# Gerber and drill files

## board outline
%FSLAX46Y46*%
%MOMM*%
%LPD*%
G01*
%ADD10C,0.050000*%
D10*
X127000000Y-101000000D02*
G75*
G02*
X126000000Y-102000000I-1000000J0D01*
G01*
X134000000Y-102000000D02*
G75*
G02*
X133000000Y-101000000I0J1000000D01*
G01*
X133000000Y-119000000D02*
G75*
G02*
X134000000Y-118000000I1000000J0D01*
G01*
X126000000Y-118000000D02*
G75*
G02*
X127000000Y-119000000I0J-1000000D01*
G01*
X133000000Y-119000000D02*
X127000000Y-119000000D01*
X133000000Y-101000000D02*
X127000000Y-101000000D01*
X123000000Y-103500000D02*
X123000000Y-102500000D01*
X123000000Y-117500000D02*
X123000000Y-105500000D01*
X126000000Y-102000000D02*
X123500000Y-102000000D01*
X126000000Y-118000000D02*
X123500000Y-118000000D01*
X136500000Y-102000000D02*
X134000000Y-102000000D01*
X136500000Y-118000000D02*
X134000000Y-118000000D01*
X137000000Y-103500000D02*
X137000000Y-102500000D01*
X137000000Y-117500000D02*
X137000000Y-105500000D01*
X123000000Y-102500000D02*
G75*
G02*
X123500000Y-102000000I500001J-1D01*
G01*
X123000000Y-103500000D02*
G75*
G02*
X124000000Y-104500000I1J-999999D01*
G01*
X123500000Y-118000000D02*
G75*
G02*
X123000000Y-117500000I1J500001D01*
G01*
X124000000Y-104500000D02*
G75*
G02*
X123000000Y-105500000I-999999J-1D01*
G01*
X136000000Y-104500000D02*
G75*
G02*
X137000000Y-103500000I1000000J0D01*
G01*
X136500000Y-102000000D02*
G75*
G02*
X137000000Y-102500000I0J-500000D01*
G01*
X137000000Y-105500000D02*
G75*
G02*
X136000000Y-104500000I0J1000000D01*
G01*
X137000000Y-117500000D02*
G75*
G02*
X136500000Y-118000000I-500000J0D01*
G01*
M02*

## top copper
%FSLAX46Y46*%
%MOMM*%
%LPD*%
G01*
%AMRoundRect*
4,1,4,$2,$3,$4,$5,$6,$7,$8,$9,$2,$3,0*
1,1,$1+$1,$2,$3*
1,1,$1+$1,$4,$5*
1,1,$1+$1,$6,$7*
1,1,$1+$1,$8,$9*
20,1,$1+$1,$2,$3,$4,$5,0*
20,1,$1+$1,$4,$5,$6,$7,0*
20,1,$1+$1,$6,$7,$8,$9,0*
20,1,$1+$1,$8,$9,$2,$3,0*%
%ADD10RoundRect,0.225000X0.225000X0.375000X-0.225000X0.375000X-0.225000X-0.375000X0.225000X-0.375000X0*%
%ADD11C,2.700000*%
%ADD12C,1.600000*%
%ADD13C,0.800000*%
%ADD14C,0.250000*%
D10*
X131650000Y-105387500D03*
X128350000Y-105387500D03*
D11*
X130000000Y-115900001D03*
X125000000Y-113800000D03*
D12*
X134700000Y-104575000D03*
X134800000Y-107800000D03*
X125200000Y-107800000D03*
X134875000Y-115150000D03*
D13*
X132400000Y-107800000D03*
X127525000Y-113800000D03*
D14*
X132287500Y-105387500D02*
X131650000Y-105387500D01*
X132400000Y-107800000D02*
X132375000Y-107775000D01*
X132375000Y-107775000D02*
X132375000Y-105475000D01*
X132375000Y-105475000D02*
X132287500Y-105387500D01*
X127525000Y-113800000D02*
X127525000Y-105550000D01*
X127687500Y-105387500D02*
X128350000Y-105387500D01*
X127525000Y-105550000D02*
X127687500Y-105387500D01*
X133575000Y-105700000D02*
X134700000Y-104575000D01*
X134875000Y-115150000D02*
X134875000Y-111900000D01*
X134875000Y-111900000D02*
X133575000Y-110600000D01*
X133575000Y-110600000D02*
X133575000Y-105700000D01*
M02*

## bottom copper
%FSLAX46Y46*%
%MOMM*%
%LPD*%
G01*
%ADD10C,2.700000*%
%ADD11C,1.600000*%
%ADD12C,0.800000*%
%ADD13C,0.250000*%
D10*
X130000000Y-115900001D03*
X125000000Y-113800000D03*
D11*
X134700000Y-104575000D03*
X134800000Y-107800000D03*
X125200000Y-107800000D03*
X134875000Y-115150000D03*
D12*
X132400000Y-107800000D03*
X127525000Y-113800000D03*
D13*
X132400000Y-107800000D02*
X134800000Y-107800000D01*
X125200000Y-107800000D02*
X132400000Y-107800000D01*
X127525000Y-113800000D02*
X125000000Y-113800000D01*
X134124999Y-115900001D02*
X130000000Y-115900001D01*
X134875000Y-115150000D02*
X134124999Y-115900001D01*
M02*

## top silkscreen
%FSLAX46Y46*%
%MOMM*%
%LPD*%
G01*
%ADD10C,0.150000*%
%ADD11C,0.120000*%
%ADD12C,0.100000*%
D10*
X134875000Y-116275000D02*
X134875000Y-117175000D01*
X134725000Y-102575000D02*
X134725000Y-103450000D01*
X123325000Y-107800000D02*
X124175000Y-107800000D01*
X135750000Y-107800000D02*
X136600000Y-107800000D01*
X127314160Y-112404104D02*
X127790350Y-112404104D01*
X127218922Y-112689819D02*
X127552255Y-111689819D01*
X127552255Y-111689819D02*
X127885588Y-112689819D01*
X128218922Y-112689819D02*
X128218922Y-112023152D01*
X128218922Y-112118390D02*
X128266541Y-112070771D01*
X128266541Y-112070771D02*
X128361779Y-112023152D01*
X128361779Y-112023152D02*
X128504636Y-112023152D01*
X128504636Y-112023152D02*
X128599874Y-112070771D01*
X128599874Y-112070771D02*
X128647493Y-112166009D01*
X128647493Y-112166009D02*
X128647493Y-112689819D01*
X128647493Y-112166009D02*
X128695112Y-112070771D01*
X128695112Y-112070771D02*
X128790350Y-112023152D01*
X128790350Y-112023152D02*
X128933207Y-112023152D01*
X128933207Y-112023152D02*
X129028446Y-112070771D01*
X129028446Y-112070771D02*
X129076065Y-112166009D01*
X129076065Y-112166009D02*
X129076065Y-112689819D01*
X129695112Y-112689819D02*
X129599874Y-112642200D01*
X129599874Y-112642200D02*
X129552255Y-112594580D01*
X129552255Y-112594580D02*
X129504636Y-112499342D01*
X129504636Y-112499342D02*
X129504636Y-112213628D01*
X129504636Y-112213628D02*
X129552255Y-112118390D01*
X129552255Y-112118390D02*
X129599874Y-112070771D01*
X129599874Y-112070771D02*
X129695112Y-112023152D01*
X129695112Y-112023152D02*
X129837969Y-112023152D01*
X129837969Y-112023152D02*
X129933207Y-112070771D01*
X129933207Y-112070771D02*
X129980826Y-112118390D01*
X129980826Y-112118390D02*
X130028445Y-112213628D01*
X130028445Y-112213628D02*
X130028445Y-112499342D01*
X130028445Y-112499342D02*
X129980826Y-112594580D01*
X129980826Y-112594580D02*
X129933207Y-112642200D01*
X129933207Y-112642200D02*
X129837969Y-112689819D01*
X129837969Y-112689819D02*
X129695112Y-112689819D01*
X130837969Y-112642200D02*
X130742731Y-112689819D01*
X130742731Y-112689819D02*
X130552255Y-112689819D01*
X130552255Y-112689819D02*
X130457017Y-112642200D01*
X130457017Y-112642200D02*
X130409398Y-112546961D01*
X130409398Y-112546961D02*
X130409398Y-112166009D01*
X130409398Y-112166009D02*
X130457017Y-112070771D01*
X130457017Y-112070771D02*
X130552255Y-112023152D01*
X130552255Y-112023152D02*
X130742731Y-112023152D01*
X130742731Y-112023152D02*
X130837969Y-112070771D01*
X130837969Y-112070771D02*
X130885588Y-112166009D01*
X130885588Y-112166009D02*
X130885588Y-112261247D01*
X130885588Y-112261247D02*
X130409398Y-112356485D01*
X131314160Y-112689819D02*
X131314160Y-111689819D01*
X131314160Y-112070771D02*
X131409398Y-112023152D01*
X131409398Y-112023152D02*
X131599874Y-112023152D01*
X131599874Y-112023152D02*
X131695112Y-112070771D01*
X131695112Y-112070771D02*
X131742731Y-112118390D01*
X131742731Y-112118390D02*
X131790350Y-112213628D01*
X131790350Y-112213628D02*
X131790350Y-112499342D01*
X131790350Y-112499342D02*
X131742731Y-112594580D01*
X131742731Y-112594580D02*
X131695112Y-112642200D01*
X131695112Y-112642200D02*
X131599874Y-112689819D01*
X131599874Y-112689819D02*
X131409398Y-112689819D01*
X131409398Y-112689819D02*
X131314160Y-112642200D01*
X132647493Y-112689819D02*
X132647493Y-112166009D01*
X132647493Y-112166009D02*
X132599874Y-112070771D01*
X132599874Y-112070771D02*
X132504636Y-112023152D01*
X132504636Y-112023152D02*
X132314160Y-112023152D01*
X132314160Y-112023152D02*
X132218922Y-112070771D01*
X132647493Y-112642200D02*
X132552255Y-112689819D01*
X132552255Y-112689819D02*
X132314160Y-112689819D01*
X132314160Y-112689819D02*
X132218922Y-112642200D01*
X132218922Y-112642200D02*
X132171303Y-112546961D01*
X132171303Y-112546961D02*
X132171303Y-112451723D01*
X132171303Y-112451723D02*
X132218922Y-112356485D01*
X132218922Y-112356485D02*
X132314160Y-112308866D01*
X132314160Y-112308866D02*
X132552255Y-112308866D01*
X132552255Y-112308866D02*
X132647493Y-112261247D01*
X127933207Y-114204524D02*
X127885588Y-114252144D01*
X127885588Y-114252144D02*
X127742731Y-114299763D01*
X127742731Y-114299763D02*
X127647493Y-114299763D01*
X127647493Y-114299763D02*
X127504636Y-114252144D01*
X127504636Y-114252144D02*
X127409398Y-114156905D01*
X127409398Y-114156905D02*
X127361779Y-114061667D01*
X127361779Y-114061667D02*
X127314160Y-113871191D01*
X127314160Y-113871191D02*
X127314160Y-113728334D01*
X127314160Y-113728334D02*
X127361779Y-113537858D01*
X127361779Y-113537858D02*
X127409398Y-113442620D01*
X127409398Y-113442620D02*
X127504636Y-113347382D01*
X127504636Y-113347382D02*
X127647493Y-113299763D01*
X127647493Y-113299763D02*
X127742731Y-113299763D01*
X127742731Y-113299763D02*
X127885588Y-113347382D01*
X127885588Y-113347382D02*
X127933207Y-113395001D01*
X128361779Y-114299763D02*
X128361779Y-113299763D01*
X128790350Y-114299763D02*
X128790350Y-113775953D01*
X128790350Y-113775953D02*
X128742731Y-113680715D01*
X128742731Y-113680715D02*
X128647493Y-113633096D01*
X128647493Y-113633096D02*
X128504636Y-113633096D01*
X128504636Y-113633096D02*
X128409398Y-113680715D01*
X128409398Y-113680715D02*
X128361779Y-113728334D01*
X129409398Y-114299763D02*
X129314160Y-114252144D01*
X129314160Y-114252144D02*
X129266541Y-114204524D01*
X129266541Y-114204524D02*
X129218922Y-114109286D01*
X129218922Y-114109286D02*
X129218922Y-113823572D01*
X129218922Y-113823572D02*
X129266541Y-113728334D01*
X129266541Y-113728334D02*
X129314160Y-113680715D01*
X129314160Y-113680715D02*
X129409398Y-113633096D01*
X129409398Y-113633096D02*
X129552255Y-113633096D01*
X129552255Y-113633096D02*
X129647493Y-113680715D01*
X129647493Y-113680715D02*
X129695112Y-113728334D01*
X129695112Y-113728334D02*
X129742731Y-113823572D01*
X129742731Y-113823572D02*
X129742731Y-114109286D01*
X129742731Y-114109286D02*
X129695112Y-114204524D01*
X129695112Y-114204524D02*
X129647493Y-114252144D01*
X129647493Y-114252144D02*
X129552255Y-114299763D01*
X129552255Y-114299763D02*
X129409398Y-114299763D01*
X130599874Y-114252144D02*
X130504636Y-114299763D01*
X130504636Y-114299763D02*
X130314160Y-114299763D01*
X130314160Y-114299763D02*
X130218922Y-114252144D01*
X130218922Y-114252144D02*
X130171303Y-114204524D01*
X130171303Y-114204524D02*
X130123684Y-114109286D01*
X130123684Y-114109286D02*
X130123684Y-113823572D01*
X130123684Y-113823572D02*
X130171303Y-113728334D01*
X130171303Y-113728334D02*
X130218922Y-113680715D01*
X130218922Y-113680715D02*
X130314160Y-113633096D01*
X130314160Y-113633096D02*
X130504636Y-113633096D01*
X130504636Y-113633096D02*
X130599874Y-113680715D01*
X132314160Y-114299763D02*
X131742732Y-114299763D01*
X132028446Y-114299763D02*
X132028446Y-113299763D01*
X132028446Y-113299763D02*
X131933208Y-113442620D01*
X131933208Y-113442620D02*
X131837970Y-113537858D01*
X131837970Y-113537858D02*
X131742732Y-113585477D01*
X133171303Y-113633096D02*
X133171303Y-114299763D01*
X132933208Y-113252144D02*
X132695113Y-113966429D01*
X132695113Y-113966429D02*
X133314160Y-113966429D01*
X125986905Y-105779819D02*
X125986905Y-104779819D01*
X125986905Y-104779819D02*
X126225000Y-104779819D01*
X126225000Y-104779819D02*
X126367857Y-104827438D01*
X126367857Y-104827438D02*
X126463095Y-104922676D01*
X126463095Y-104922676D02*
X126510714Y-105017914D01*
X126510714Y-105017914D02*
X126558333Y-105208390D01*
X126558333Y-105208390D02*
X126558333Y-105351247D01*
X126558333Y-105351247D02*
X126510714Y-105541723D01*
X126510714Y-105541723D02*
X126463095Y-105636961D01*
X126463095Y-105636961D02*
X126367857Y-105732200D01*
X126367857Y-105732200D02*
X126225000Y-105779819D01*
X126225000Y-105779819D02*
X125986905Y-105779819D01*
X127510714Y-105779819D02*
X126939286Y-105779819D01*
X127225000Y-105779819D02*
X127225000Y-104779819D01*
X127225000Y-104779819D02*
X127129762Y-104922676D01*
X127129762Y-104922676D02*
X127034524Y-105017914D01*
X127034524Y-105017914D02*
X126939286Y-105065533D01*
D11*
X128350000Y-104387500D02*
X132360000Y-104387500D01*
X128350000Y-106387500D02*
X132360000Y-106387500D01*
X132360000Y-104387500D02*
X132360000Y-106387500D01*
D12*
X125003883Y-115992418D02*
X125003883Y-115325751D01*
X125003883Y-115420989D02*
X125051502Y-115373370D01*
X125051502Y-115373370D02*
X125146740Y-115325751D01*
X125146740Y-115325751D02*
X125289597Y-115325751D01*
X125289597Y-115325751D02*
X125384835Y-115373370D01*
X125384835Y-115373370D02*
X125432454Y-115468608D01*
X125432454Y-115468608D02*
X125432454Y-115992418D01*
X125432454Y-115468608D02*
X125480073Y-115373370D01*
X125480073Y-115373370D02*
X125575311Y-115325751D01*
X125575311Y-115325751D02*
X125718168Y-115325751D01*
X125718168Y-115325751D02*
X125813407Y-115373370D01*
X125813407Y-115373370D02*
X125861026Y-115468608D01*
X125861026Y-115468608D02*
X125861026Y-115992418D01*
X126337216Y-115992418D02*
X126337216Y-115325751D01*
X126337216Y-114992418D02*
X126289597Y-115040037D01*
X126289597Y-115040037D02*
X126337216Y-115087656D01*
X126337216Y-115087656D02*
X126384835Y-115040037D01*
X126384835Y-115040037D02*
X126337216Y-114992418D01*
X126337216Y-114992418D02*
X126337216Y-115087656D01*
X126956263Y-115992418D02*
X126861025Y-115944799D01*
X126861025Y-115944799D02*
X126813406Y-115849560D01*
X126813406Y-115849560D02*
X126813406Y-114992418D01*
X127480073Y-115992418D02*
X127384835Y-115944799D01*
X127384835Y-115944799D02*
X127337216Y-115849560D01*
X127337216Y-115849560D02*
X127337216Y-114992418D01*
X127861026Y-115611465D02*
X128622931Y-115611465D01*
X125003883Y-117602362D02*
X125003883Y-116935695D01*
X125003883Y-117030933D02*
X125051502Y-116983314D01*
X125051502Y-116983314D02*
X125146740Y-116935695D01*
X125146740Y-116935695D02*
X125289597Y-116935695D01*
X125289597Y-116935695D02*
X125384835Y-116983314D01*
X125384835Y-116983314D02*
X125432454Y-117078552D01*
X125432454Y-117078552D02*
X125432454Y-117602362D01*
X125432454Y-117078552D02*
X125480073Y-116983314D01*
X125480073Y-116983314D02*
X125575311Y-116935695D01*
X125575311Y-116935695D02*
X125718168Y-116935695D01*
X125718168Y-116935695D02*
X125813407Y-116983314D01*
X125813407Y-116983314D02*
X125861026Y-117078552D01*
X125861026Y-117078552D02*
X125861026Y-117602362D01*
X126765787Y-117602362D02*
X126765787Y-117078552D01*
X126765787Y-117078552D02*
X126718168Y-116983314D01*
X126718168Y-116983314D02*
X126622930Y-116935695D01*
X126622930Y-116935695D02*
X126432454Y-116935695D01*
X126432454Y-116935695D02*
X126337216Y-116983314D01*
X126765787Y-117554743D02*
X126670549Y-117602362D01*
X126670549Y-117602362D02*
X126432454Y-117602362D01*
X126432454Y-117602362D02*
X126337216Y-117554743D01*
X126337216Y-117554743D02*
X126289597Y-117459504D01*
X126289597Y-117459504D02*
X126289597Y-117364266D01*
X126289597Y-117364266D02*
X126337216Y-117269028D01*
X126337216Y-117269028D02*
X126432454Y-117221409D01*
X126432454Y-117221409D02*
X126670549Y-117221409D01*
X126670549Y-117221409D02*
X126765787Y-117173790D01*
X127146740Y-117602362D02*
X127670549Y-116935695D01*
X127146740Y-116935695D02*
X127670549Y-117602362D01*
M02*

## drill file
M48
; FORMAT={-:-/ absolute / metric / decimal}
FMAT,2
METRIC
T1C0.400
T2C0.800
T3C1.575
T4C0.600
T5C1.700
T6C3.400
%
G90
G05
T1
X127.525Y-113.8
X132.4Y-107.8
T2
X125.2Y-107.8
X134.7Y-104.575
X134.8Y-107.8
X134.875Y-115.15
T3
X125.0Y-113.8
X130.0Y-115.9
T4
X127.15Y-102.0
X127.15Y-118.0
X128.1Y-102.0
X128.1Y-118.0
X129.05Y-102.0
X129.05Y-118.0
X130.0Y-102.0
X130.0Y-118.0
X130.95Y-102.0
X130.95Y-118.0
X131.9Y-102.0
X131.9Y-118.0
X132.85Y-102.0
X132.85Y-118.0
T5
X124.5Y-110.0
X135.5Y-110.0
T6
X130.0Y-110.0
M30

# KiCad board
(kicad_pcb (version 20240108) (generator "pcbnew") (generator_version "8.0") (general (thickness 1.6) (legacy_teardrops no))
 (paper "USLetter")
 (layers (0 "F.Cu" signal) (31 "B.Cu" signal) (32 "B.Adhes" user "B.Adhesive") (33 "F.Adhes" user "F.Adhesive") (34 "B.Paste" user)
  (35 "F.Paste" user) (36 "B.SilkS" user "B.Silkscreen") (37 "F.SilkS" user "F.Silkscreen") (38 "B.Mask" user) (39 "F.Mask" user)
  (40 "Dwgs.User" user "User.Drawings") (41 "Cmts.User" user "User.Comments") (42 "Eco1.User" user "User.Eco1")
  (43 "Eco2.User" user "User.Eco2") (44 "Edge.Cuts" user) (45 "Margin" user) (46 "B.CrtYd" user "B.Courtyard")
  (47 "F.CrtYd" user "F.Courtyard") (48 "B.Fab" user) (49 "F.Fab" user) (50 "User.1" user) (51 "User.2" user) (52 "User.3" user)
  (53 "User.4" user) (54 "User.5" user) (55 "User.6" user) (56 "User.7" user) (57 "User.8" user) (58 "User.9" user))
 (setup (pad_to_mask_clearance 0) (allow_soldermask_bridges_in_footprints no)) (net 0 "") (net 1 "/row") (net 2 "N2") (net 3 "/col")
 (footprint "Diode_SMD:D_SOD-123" (layer "F.Cu") (at 130 105.3875 180)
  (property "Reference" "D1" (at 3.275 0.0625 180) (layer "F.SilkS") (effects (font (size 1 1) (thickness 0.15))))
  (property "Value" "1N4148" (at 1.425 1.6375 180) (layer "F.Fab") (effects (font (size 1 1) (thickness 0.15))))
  (fp_line (start 1.65 1) (end -2.36 1) (stroke (width 0.12) (type solid)) (layer "F.SilkS"))
  (fp_line (start 1.65 -1) (end -2.36 -1) (stroke (width 0.12) (type solid)) (layer "F.SilkS"))
  (fp_line (start -2.36 1) (end -2.36 -1) (stroke (width 0.12) (type solid)) (layer "F.SilkS"))
  (pad "1" smd roundrect (at -1.65 0 180) (size 0.9 1.2) (layers "F.Cu" "F.Paste" "F.Mask") (roundrect_rratio 0.25) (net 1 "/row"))
  (pad "2" smd roundrect (at 1.65 0 180) (size 0.9 1.2) (layers "F.Cu" "F.Paste" "F.Mask") (roundrect_rratio 0.25) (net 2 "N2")))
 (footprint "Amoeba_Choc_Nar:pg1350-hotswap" (layer "F.Cu") (at 130 110)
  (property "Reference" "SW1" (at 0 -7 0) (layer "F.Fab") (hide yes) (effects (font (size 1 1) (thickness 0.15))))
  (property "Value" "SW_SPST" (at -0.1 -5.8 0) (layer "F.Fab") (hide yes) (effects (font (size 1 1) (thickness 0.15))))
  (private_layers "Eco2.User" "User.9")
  (fp_line (start -7 -6.5) (end -7 -7.5) (stroke (width 0.05) (type solid)) (layer "Edge.Cuts"))
  (fp_line (start -7 7.5) (end -7 -4.5) (stroke (width 0.05) (type solid)) (layer "Edge.Cuts"))
  (fp_line (start -4 -8) (end -6.5 -8) (stroke (width 0.05) (type solid)) (layer "Edge.Cuts"))
  (fp_line (start -4 8) (end -6.5 8) (stroke (width 0.05) (type solid)) (layer "Edge.Cuts"))
  (fp_line (start 6.5 -8) (end 4 -8) (stroke (width 0.05) (type solid)) (layer "Edge.Cuts"))
  (fp_line (start 6.5 8) (end 4 8) (stroke (width 0.05) (type solid)) (layer "Edge.Cuts"))
  (fp_line (start 7 -6.5) (end 7 -7.5) (stroke (width 0.05) (type solid)) (layer "Edge.Cuts"))
  (fp_line (start 7 7.5) (end 7 -4.5) (stroke (width 0.05) (type solid)) (layer "Edge.Cuts"))
  (fp_arc (start -7 -7.5) (mid -6.853553 -7.853553) (end -6.5 -8) (stroke (width 0.05) (type default)) (layer "Edge.Cuts"))
  (fp_arc (start -7 -6.5) (mid -6.292893 -6.207107) (end -6 -5.5) (stroke (width 0.05) (type default)) (layer "Edge.Cuts"))
  (fp_arc (start -6.5 8) (mid -6.853553 7.853553) (end -7 7.5) (stroke (width 0.05) (type default)) (layer "Edge.Cuts"))
  (fp_arc (start -6 -5.5) (mid -6.292893 -4.792893) (end -7 -4.5) (stroke (width 0.05) (type default)) (layer "Edge.Cuts"))
  (fp_arc (start 6 -5.5) (mid 6.292893 -6.207107) (end 7 -6.5) (stroke (width 0.05) (type default)) (layer "Edge.Cuts"))
  (fp_arc (start 6.5 -8) (mid 6.853553 -7.853553) (end 7 -7.5) (stroke (width 0.05) (type default)) (layer "Edge.Cuts"))
  (fp_arc (start 7 -4.5) (mid 6.292893 -4.792893) (end 6 -5.5) (stroke (width 0.05) (type default)) (layer "Edge.Cuts"))
  (fp_arc (start 7 7.5) (mid 6.853553 7.853553) (end 6.5 8) (stroke (width 0.05) (type default)) (layer "Edge.Cuts"))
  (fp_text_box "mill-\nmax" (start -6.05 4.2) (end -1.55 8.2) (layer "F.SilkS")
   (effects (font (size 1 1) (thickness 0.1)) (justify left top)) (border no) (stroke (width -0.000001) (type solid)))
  (pad "" np_thru_hole circle (at -5.5 0 180) (size 1.7 1.7) (drill 1.7) (layers "*.Cu" "*.Mask"))
  (pad "" np_thru_hole circle (at 0 0 180) (size 3.4 3.4) (drill 3.4) (layers "*.Cu" "*.Mask"))
  (pad "" np_thru_hole circle (at 5.5 0 180) (size 1.7 1.7) (drill 1.7) (layers "*.Cu" "*.Mask"))
  (pad "1" thru_hole circle (at 0 5.900001 180) (size 2.7 2.7) (drill 1.5748) (layers "*.Cu" "*.Mask") (remove_unused_layers no)
   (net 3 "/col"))
  (pad "2" thru_hole circle (at -5 3.8 180) (size 2.7 2.7) (drill 1.5748) (layers "*.Cu" "*.Mask") (remove_unused_layers no) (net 2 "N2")))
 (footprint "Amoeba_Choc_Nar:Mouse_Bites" (layer "F.Cu") (at 130 118)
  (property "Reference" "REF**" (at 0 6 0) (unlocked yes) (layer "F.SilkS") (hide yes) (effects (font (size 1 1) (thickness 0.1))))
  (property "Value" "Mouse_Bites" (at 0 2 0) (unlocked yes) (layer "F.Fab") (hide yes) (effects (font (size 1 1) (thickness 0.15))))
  (pad "" np_thru_hole circle (at -2.85 0) (size 0.6 0.6) (drill 0.6) (layers "*.Mask"))
  (pad "" np_thru_hole circle (at -1.9 0) (size 0.6 0.6) (drill 0.6) (layers "*.Mask"))
  (pad "" np_thru_hole circle (at -0.95 0) (size 0.6 0.6) (drill 0.6) (layers "*.Mask"))
  (pad "" np_thru_hole circle (at 0 0) (size 0.6 0.6) (drill 0.6) (layers "*.Mask"))
  (pad "" np_thru_hole circle (at 0.95 0) (size 0.6 0.6) (drill 0.6) (layers "*.Mask"))
  (pad "" np_thru_hole circle (at 1.9 0) (size 0.6 0.6) (drill 0.6) (layers "*.Mask"))
  (pad "" np_thru_hole circle (at 2.85 0) (size 0.6 0.6) (drill 0.6) (layers "*.Mask")))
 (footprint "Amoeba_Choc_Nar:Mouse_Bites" (layer "F.Cu") (at 130 102)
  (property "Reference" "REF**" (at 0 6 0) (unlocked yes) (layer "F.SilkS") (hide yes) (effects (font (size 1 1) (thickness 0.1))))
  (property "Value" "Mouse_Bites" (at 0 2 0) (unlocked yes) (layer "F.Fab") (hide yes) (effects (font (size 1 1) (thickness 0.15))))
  (pad "" np_thru_hole circle (at -2.85 0) (size 0.6 0.6) (drill 0.6) (layers "*.Mask"))
  (pad "" np_thru_hole circle (at -1.9 0) (size 0.6 0.6) (drill 0.6) (layers "*.Mask"))
  (pad "" np_thru_hole circle (at -0.95 0) (size 0.6 0.6) (drill 0.6) (layers "*.Mask"))
  (pad "" np_thru_hole circle (at 0 0) (size 0.6 0.6) (drill 0.6) (layers "*.Mask"))
  (pad "" np_thru_hole circle (at 0.95 0) (size 0.6 0.6) (drill 0.6) (layers "*.Mask"))
  (pad "" np_thru_hole circle (at 1.9 0) (size 0.6 0.6) (drill 0.6) (layers "*.Mask"))
  (pad "" np_thru_hole circle (at 2.85 0) (size 0.6 0.6) (drill 0.6) (layers "*.Mask")))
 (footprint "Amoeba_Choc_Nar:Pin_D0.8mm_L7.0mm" (layer "B.Cu") (at 134.7 104.575 180)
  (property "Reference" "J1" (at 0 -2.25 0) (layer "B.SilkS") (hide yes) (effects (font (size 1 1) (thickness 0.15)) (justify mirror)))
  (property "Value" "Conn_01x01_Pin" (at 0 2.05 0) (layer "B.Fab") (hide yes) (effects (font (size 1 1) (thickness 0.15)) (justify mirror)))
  (pad "1" thru_hole circle (at 0 0 180) (size 1.6 1.6) (drill 0.8) (layers "*.Cu" "*.Mask") (remove_unused_layers no) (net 3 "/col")))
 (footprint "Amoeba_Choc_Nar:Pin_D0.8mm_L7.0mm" (layer "B.Cu") (at 134.8 107.8 180)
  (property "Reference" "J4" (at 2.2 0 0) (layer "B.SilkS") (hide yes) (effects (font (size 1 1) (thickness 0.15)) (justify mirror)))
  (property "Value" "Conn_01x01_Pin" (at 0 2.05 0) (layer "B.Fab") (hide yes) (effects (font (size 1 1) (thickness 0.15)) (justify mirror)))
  (pad "1" thru_hole circle (at 0 0 180) (size 1.6 1.6) (drill 0.8) (layers "*.Cu" "*.Mask") (remove_unused_layers no) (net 1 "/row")))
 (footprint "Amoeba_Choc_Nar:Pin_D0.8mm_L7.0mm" (layer "B.Cu") (at 125.2 107.8 180)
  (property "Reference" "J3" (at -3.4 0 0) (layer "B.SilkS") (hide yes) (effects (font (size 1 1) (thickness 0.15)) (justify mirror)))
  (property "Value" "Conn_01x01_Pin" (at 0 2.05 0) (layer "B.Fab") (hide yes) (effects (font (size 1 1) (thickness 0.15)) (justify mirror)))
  (pad "1" thru_hole circle (at 0 0 180) (size 1.6 1.6) (drill 0.8) (layers "*.Cu" "*.Mask") (remove_unused_layers no) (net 1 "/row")))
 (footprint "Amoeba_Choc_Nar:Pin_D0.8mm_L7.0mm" (layer "B.Cu") (at 134.875 115.15 180)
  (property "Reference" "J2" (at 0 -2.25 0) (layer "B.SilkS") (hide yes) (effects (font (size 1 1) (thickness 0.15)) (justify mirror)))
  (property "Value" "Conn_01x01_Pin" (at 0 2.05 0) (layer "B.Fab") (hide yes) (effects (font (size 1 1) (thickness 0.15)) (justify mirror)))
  (pad "1" thru_hole circle (at 0 0 180) (size 1.6 1.6) (drill 0.8) (layers "*.Cu" "*.Mask") (remove_unused_layers no) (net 3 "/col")))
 (gr_line (start 134.875 116.275) (end 134.875 117.175) (stroke (width 0.15) (type default)) (layer "F.SilkS"))
 (gr_line (start 134.725 102.575) (end 134.725 103.45) (stroke (width 0.15) (type default)) (layer "F.SilkS"))
 (gr_line (start 123.325 107.8) (end 124.175 107.8) (stroke (width 0.15) (type default)) (layer "F.SilkS"))
 (gr_line (start 135.75 107.8) (end 136.6 107.8) (stroke (width 0.15) (type default)) (layer "F.SilkS"))
 (gr_arc (start 127 101) (mid 126.707107 101.707107) (end 126 102) (stroke (width 0.05) (type default)) (layer "Edge.Cuts"))
 (gr_arc (start 134 102) (mid 133.292893 101.707107) (end 133 101) (stroke (width 0.05) (type default)) (layer "Edge.Cuts"))
 (gr_arc (start 133 119) (mid 133.292893 118.292893) (end 134 118) (stroke (width 0.05) (type default)) (layer "Edge.Cuts"))
 (gr_arc (start 126 118) (mid 126.707107 118.292893) (end 127 119) (stroke (width 0.05) (type default)) (layer "Edge.Cuts"))
 (gr_line (start 133 119) (end 127 119) (stroke (width 0.05) (type default)) (layer "Edge.Cuts"))
 (gr_line (start 133 101) (end 127 101) (stroke (width 0.05) (type default)) (layer "Edge.Cuts"))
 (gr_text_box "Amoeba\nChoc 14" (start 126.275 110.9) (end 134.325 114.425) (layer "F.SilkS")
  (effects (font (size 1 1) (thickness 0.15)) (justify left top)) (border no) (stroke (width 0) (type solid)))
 (segment (start 132.2875 105.3875) (end 131.65 105.3875) (width 0.25) (layer "F.Cu") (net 1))
 (segment (start 132.4 107.8) (end 132.375 107.775) (width 0.25) (layer "F.Cu") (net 1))
 (segment (start 132.375 107.775) (end 132.375 105.475) (width 0.25) (layer "F.Cu") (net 1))
 (segment (start 132.375 105.475) (end 132.2875 105.3875) (width 0.25) (layer "F.Cu") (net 1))
 (via (at 132.4 107.8) (size 0.8) (drill 0.4) (layers "F.Cu" "B.Cu") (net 1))
 (segment (start 132.4 107.8) (end 134.8 107.8) (width 0.25) (layer "B.Cu") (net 1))
 (segment (start 125.2 107.8) (end 132.4 107.8) (width 0.25) (layer "B.Cu") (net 1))
 (segment (start 127.525 113.8) (end 127.525 105.55) (width 0.25) (layer "F.Cu") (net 2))
 (segment (start 127.6875 105.3875) (end 128.35 105.3875) (width 0.25) (layer "F.Cu") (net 2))
 (segment (start 127.525 105.55) (end 127.6875 105.3875) (width 0.25) (layer "F.Cu") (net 2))
 (via (at 127.525 113.8) (size 0.8) (drill 0.4) (layers "F.Cu" "B.Cu") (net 2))
 (segment (start 127.525 113.8) (end 125 113.8) (width 0.25) (layer "B.Cu") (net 2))
 (segment (start 133.575 105.7) (end 134.7 104.575) (width 0.25) (layer "F.Cu") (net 3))
 (segment (start 134.875 115.15) (end 134.875 111.9) (width 0.25) (layer "F.Cu") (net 3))
 (segment (start 134.875 111.9) (end 133.575 110.6) (width 0.25) (layer "F.Cu") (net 3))
 (segment (start 133.575 110.6) (end 133.575 105.7) (width 0.25) (layer "F.Cu") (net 3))
 (segment (start 134.124999 115.900001) (end 130 115.900001) (width 0.25) (layer "B.Cu") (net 3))
 (segment (start 134.875 115.15) (end 134.124999 115.900001) (width 0.25) (layer "B.Cu") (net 3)))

